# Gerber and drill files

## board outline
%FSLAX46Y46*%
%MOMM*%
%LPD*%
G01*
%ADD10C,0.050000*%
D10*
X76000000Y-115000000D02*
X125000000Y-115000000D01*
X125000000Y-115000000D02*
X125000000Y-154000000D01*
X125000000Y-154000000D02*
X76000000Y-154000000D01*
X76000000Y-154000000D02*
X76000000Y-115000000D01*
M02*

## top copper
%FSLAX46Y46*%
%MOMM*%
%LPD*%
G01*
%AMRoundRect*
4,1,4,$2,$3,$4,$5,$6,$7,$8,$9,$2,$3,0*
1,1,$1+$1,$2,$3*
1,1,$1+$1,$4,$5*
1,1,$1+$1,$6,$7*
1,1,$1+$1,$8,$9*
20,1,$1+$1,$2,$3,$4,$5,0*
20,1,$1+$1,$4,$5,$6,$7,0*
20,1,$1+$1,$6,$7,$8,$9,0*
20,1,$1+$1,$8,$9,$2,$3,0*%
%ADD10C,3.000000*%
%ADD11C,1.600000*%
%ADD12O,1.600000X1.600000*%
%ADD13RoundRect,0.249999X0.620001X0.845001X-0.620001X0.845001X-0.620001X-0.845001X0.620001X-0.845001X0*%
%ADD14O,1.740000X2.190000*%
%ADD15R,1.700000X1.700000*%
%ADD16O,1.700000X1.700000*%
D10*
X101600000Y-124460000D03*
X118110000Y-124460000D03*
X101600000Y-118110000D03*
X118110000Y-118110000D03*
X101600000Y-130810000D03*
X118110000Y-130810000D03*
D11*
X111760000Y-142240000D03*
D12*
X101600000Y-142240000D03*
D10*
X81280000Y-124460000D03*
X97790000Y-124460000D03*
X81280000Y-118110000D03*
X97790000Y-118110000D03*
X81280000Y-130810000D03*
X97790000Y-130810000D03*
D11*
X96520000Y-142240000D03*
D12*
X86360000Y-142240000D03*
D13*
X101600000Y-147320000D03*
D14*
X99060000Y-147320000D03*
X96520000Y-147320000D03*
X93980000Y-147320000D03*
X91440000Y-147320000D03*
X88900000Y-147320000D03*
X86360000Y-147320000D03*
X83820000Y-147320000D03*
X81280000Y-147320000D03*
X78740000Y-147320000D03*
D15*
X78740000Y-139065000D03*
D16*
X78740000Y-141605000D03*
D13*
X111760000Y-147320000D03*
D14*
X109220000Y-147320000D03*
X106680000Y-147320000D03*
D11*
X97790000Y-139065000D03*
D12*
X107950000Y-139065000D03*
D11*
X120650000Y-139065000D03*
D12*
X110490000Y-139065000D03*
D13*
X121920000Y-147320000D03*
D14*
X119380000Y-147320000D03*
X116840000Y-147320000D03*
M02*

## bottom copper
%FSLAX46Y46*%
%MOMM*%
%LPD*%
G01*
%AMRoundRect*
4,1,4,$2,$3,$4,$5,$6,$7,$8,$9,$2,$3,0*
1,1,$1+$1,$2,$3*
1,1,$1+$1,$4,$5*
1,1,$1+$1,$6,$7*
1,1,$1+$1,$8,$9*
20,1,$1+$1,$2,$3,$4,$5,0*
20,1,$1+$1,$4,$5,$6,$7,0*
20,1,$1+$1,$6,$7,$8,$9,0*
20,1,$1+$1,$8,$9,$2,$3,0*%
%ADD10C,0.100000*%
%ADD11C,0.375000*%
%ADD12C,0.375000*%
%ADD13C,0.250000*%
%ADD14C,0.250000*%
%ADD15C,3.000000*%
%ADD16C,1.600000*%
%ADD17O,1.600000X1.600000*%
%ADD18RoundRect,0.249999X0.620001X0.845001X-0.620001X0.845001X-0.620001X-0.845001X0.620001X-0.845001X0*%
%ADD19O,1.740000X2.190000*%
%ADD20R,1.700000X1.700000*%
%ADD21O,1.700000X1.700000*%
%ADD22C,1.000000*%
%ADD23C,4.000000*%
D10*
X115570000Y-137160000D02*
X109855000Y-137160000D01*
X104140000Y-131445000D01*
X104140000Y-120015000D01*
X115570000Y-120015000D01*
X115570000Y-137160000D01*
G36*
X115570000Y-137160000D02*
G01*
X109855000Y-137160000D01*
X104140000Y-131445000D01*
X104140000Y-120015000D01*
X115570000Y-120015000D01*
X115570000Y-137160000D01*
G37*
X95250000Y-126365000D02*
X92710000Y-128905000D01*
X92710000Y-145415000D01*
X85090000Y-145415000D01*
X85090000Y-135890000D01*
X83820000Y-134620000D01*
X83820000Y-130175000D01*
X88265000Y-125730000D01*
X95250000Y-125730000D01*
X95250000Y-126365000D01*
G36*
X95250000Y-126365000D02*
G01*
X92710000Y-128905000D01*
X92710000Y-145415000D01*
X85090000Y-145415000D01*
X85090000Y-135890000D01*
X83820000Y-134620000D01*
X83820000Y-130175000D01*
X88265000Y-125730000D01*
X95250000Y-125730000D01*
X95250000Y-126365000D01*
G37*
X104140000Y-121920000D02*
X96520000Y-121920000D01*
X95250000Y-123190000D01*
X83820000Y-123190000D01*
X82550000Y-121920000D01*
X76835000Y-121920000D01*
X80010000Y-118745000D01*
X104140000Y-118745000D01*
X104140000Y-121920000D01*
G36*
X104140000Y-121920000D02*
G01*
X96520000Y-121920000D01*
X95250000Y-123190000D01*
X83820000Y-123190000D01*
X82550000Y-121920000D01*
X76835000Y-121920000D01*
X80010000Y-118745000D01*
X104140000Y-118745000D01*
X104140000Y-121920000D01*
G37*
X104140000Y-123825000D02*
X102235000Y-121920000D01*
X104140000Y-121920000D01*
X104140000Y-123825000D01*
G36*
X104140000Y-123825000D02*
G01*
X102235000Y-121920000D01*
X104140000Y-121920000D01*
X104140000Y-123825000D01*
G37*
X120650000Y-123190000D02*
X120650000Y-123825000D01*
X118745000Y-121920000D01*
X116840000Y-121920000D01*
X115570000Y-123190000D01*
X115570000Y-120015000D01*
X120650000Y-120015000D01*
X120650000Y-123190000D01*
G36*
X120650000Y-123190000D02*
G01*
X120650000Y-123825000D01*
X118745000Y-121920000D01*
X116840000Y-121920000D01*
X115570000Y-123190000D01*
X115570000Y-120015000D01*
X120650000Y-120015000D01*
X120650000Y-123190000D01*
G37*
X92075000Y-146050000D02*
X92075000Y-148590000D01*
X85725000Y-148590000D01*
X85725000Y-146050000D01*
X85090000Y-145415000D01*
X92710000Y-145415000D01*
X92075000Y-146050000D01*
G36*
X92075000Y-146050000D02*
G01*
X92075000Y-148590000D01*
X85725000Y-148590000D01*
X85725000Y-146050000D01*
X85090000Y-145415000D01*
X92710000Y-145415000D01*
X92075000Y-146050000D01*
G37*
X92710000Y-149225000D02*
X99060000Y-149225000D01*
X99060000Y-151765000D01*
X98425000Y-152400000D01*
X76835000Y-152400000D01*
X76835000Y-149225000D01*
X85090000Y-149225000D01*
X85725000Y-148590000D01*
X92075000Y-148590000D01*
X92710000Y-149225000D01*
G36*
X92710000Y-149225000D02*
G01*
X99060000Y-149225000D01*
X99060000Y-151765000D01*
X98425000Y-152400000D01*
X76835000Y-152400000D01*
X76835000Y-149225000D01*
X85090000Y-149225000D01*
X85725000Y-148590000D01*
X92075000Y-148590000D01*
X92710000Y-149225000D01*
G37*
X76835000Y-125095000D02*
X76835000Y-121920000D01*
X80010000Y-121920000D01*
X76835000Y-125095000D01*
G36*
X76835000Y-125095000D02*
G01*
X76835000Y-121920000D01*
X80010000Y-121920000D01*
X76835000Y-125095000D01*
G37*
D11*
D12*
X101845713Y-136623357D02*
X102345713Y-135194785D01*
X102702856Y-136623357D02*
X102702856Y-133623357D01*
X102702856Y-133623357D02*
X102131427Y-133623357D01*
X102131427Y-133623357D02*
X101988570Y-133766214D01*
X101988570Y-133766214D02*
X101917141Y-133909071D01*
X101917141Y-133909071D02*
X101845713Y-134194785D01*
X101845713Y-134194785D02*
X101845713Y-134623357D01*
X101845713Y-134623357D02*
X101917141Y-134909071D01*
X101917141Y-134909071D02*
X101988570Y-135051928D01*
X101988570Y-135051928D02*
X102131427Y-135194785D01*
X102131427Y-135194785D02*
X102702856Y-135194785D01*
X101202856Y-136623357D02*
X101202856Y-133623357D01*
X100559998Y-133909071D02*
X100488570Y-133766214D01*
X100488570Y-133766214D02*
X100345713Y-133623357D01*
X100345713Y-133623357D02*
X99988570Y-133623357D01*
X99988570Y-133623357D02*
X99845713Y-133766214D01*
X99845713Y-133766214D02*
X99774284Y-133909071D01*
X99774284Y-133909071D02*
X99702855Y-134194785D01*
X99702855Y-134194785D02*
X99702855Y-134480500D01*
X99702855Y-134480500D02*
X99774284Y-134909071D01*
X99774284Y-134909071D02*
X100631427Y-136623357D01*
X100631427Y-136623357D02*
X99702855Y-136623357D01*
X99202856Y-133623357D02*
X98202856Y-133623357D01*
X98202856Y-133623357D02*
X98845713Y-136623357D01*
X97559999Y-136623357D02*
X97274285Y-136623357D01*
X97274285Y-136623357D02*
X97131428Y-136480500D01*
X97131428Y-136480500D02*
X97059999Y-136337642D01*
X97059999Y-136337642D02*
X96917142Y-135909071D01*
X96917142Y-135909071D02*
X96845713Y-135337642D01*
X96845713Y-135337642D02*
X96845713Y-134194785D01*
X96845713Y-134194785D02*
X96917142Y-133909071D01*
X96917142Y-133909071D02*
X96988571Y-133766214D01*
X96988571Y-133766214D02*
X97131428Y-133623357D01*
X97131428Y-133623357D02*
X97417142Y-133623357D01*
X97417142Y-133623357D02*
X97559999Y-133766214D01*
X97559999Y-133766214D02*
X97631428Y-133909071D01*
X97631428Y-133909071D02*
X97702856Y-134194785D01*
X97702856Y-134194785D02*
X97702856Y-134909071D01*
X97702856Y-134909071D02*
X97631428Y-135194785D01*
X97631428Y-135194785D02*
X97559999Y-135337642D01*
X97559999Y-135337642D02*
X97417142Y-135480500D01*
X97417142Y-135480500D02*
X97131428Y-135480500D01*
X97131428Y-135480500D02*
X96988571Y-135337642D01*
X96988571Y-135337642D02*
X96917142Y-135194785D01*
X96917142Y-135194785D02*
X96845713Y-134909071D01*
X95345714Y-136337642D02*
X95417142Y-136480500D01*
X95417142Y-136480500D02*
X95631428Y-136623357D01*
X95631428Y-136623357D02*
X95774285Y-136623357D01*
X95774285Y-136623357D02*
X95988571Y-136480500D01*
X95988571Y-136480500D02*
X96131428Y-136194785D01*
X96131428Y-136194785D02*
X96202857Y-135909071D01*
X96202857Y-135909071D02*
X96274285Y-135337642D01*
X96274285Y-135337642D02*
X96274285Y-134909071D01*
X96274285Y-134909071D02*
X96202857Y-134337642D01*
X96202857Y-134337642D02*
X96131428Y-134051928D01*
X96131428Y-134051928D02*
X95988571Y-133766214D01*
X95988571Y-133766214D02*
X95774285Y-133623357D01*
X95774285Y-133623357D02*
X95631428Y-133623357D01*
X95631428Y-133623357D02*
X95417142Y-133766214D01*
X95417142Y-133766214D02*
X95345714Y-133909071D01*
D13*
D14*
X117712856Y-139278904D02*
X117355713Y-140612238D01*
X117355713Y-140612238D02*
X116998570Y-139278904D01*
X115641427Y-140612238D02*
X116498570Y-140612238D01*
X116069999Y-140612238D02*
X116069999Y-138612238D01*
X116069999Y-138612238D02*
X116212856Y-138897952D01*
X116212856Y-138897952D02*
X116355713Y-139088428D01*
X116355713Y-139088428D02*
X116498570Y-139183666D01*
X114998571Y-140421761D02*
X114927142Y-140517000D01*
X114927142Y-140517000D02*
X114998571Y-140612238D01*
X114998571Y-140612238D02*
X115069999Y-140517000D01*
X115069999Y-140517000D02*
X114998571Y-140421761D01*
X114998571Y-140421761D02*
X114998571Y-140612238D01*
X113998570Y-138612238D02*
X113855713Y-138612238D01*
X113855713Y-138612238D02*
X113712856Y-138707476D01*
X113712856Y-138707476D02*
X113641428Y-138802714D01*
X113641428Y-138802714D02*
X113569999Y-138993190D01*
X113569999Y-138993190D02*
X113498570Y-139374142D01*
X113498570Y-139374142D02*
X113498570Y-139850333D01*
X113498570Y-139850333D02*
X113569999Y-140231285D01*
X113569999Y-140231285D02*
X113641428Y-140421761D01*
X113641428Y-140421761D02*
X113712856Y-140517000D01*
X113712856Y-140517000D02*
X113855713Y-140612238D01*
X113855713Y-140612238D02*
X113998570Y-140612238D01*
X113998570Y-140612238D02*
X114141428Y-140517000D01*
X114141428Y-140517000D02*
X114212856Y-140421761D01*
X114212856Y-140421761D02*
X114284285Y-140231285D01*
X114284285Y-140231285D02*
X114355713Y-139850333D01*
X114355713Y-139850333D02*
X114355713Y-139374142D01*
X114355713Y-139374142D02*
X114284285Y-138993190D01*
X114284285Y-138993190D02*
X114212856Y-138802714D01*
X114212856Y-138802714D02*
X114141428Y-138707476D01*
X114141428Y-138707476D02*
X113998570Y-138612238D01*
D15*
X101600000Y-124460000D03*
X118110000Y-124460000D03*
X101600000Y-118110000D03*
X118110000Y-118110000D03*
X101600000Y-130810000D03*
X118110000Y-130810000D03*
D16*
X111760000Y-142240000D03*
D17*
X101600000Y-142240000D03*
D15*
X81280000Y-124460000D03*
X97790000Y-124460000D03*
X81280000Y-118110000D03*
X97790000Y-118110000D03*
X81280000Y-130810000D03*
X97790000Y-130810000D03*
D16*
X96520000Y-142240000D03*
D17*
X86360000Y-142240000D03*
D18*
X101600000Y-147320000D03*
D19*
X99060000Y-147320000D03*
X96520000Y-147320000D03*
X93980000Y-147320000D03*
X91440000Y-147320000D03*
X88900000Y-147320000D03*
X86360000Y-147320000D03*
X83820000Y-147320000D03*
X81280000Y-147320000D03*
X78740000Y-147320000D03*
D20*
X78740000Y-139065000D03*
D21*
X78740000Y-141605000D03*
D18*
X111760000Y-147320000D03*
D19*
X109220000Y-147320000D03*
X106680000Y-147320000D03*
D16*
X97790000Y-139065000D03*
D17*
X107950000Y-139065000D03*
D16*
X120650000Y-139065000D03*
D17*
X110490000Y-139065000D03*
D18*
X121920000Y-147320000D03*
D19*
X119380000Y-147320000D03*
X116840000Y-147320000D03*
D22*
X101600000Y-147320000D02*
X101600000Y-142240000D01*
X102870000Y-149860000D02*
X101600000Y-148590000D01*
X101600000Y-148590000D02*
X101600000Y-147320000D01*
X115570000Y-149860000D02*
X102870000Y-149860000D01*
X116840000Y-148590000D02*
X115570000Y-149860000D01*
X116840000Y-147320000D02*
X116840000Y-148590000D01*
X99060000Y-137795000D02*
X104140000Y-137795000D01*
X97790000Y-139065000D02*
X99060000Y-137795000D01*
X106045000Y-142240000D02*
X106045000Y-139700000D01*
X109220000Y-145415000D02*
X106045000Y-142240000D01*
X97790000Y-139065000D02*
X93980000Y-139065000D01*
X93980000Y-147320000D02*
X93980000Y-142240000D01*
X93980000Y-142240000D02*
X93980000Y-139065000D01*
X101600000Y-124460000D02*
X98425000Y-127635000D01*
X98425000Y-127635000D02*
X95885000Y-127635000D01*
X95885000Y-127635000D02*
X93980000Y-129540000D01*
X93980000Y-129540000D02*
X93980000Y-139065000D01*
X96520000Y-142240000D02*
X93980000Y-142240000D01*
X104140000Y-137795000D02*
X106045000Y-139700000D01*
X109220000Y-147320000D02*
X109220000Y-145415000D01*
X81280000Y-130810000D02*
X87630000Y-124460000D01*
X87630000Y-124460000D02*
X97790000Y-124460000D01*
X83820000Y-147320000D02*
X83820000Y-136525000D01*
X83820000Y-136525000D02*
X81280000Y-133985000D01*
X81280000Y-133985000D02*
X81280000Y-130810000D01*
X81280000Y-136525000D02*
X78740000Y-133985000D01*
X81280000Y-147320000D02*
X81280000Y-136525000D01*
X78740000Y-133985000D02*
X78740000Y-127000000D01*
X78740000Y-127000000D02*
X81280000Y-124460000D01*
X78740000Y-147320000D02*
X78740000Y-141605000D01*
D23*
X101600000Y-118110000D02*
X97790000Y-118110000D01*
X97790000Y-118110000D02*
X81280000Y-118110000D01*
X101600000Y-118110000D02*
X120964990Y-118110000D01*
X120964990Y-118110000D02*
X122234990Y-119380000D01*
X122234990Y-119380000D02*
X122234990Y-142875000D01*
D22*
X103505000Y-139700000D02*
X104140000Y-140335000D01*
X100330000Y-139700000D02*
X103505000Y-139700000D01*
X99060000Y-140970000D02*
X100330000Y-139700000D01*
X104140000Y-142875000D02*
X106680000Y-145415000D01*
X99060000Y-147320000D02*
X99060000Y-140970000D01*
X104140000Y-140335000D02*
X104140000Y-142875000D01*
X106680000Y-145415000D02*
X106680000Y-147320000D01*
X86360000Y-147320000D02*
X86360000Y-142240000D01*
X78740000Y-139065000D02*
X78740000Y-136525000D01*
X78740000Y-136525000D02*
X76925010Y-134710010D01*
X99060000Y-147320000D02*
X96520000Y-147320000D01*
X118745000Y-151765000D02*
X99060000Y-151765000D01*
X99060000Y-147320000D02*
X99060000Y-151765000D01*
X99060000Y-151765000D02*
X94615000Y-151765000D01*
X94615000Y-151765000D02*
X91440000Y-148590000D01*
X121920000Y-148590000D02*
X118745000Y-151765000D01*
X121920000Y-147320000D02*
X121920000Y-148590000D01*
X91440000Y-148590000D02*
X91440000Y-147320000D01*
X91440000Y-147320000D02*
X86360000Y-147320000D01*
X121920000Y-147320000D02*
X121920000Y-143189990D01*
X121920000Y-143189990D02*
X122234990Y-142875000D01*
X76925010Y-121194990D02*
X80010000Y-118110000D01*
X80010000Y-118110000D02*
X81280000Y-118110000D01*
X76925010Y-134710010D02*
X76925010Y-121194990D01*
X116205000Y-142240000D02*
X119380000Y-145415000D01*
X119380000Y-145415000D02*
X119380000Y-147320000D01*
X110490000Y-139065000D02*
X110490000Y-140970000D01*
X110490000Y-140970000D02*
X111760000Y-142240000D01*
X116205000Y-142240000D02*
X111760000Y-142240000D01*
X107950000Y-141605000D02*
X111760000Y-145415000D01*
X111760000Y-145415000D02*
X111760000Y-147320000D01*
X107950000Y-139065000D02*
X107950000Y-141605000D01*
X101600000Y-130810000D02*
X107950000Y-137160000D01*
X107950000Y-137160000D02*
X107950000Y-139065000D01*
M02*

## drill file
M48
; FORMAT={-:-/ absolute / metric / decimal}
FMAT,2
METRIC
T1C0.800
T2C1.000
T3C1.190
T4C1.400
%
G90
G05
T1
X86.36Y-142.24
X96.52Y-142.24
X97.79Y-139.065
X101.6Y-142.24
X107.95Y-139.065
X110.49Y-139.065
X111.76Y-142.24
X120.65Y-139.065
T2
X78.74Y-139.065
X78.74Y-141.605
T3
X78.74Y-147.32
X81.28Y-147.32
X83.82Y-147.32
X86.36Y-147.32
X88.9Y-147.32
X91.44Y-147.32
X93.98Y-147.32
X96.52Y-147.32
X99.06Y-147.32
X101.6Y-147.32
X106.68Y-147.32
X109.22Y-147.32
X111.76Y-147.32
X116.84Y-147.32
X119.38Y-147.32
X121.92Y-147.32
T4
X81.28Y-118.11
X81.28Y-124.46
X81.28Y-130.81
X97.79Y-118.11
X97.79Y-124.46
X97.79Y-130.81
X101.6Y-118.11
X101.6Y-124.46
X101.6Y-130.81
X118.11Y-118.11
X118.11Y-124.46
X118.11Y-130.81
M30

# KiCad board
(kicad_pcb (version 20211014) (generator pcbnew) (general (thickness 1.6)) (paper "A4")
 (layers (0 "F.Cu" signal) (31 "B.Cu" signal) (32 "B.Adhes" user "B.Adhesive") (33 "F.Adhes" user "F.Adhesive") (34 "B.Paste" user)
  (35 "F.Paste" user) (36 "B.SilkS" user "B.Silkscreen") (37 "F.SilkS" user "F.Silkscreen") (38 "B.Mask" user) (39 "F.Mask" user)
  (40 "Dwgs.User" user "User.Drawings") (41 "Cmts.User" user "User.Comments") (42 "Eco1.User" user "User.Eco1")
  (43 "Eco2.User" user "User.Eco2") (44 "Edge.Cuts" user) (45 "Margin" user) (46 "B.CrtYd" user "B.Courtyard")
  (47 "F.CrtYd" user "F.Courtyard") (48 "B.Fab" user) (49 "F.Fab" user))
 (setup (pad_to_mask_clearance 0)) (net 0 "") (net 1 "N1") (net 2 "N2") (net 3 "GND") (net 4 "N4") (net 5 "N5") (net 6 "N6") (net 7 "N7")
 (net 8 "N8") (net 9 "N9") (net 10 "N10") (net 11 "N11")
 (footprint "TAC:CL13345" (layer "F.Cu") (at 109.855 118.11 90)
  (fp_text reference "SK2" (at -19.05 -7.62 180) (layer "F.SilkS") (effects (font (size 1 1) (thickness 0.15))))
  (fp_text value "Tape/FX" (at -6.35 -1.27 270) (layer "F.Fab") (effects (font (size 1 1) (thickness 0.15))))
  (pad "R" thru_hole circle locked (at -6.35 -8.255 180) (size 3 3) (drill 1.4) (layers *.Cu *.Mask) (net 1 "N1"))
  (pad "RN" thru_hole circle locked (at -6.35 8.255 180) (size 3 3) (drill 1.4) (layers *.Cu *.Mask) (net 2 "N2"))
  (pad "S" thru_hole circle locked (at 0 -8.255 180) (size 3 3) (drill 1.4) (layers *.Cu *.Mask) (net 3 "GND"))
  (pad "SN" thru_hole circle locked (at 0 8.255 180) (size 3 3) (drill 1.4) (layers *.Cu *.Mask) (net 3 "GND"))
  (pad "T" thru_hole circle locked (at -12.7 -8.255 180) (size 3 3) (drill 1.4) (layers *.Cu *.Mask) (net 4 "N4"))
  (pad "TN" thru_hole circle locked (at -12.7 8.255 180) (size 3 3) (drill 1.4) (layers *.Cu *.Mask) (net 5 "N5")))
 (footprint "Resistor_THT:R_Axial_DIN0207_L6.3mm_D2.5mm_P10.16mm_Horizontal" (layer "F.Cu") (at 111.76 142.24 180)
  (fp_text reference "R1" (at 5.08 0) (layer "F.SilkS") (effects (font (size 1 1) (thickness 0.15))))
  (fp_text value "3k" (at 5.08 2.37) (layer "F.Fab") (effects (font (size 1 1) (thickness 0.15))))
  (pad "1" thru_hole circle locked (at 0 0 180) (size 1.6 1.6) (drill 0.8) (layers *.Cu *.Mask) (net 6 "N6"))
  (pad "2" thru_hole oval locked (at 10.16 0 180) (size 1.6 1.6) (drill 0.8) (layers *.Cu *.Mask) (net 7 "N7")))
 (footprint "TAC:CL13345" (layer "F.Cu") (at 89.535 118.11 90)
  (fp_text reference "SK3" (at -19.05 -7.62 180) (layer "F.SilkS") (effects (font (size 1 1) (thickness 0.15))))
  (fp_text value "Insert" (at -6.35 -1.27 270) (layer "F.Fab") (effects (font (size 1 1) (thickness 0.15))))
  (pad "R" thru_hole circle locked (at -6.35 -8.255 180) (size 3 3) (drill 1.4) (layers *.Cu *.Mask) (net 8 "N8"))
  (pad "RN" thru_hole circle locked (at -6.35 8.255 180) (size 3 3) (drill 1.4) (layers *.Cu *.Mask) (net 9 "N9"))
  (pad "S" thru_hole circle locked (at 0 -8.255 180) (size 3 3) (drill 1.4) (layers *.Cu *.Mask) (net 3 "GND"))
  (pad "SN" thru_hole circle locked (at 0 8.255 180) (size 3 3) (drill 1.4) (layers *.Cu *.Mask) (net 3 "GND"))
  (pad "T" thru_hole circle locked (at -12.7 -8.255 180) (size 3 3) (drill 1.4) (layers *.Cu *.Mask) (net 9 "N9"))
  (pad "TN" thru_hole circle locked (at -12.7 8.255 180) (size 3 3) (drill 1.4) (layers *.Cu *.Mask) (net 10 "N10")))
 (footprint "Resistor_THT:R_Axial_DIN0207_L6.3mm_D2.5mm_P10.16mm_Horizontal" (layer "F.Cu") (at 96.52 142.24 180)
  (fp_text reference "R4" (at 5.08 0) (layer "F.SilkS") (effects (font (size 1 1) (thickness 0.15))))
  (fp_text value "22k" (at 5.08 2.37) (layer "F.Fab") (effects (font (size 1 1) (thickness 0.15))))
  (pad "1" thru_hole circle locked (at 0 0 180) (size 1.6 1.6) (drill 0.8) (layers *.Cu *.Mask) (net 1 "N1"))
  (pad "2" thru_hole oval locked (at 10.16 0 180) (size 1.6 1.6) (drill 0.8) (layers *.Cu *.Mask) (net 3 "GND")))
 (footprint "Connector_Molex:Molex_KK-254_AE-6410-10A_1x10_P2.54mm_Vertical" (layer "F.Cu") (at 101.6 147.32 180)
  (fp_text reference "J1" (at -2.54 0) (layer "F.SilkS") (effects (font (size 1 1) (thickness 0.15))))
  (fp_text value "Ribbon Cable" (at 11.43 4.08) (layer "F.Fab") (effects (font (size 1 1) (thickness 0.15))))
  (pad "1" thru_hole roundrect locked (at 0 0 180) (size 1.74 2.19) (drill 1.19) (layers *.Cu *.Mask) (roundrect_rratio 0.1436775862)
   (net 7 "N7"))
  (pad "2" thru_hole oval locked (at 2.54 0 180) (size 1.74 2.19) (drill 1.19) (layers *.Cu *.Mask) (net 3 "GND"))
  (pad "3" thru_hole oval locked (at 5.08 0 180) (size 1.74 2.19) (drill 1.19) (layers *.Cu *.Mask) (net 3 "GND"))
  (pad "4" thru_hole oval locked (at 7.62 0 180) (size 1.74 2.19) (drill 1.19) (layers *.Cu *.Mask) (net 1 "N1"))
  (pad "5" thru_hole oval locked (at 10.16 0 180) (size 1.74 2.19) (drill 1.19) (layers *.Cu *.Mask) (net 3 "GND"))
  (pad "6" thru_hole oval locked (at 12.7 0 180) (size 1.74 2.19) (drill 1.19) (layers *.Cu *.Mask) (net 3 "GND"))
  (pad "7" thru_hole oval locked (at 15.24 0 180) (size 1.74 2.19) (drill 1.19) (layers *.Cu *.Mask) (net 3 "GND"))
  (pad "8" thru_hole oval locked (at 17.78 0 180) (size 1.74 2.19) (drill 1.19) (layers *.Cu *.Mask) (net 9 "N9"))
  (pad "9" thru_hole oval locked (at 20.32 0 180) (size 1.74 2.19) (drill 1.19) (layers *.Cu *.Mask) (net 8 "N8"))
  (pad "10" thru_hole oval locked (at 22.86 0 180) (size 1.74 2.19) (drill 1.19) (layers *.Cu *.Mask) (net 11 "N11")))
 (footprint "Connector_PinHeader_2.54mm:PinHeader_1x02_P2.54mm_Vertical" (layer "F.Cu") (at 78.74 139.065)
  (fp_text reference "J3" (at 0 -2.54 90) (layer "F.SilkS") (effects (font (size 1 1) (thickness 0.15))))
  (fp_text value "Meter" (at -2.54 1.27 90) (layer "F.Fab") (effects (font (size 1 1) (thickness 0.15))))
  (pad "1" thru_hole rect locked (at 0 0) (size 1.7 1.7) (drill 1) (layers *.Cu *.Mask) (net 3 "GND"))
  (pad "2" thru_hole oval locked (at 0 2.54) (size 1.7 1.7) (drill 1) (layers *.Cu *.Mask) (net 11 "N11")))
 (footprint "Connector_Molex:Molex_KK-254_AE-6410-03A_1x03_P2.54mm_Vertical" (layer "F.Cu") (at 111.76 147.32 180)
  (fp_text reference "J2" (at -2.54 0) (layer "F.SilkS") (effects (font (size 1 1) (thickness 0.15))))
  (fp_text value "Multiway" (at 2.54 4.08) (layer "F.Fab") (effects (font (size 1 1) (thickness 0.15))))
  (pad "1" thru_hole roundrect locked (at 0 0 180) (size 1.74 2.19) (drill 1.19) (layers *.Cu *.Mask) (roundrect_rratio 0.1436775862)
   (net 4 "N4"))
  (pad "2" thru_hole oval locked (at 2.54 0 180) (size 1.74 2.19) (drill 1.19) (layers *.Cu *.Mask) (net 1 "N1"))
  (pad "3" thru_hole oval locked (at 5.08 0 180) (size 1.74 2.19) (drill 1.19) (layers *.Cu *.Mask) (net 3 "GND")))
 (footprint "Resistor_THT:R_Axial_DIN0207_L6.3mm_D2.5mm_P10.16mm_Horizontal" (layer "F.Cu") (at 97.79 139.065)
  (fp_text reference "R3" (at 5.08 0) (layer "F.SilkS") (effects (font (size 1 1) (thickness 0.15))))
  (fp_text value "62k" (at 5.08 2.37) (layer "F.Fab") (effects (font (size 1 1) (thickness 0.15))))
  (pad "1" thru_hole circle locked (at 0 0) (size 1.6 1.6) (drill 0.8) (layers *.Cu *.Mask) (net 1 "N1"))
  (pad "2" thru_hole oval locked (at 10.16 0) (size 1.6 1.6) (drill 0.8) (layers *.Cu *.Mask) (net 4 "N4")))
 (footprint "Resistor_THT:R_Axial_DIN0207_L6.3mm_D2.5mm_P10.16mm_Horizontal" (layer "F.Cu") (at 120.65 139.065 180)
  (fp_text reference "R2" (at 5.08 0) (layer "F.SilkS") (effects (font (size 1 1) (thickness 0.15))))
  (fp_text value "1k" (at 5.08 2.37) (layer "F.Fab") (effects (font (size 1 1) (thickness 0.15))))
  (pad "1" thru_hole circle locked (at 0 0 180) (size 1.6 1.6) (drill 0.8) (layers *.Cu *.Mask) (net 3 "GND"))
  (pad "2" thru_hole oval locked (at 10.16 0 180) (size 1.6 1.6) (drill 0.8) (layers *.Cu *.Mask) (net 6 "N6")))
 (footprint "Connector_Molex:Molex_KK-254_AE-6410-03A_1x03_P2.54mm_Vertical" (layer "F.Cu") (at 121.92 147.32 180)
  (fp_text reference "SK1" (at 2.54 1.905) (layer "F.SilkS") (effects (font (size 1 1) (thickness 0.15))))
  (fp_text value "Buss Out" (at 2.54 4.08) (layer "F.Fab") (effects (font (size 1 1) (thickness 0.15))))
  (pad "1" thru_hole roundrect locked (at 0 0 180) (size 1.74 2.19) (drill 1.19) (layers *.Cu *.Mask) (roundrect_rratio 0.1436775862)
   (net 3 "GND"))
  (pad "2" thru_hole oval locked (at 2.54 0 180) (size 1.74 2.19) (drill 1.19) (layers *.Cu *.Mask) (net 6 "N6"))
  (pad "3" thru_hole oval locked (at 5.08 0 180) (size 1.74 2.19) (drill 1.19) (layers *.Cu *.Mask) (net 7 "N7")))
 (gr_poly
  (pts (xy 115.57 137.16) (xy 109.855 137.16) (xy 104.14 131.445) (xy 104.14 120.015) (xy 115.57 120.015)) (layer "B.Cu") (width 0.1)
  (fill solid))
 (gr_poly
  (pts (xy 95.25 126.365) (xy 92.71 128.905) (xy 92.71 145.415) (xy 85.09 145.415) (xy 85.09 135.89) (xy 83.82 134.62) (xy 83.82 130.175)
   (xy 88.265 125.73) (xy 95.25 125.73))
  (layer "B.Cu") (width 0.1) (fill solid))
 (gr_poly
  (pts (xy 104.14 121.92) (xy 96.52 121.92) (xy 95.25 123.19) (xy 83.82 123.19) (xy 82.55 121.92) (xy 76.835 121.92) (xy 80.01 118.745)
   (xy 104.14 118.745))
  (layer "B.Cu") (width 0.1) (fill solid))
 (gr_poly (pts (xy 104.14 123.825) (xy 102.235 121.92) (xy 104.14 121.92)) (layer "B.Cu") (width 0.1) (fill solid))
 (gr_poly
  (pts (xy 120.65 123.19) (xy 120.65 123.825) (xy 118.745 121.92) (xy 116.84 121.92) (xy 115.57 123.19) (xy 115.57 120.015)
   (xy 120.65 120.015))
  (layer "B.Cu") (width 0.1) (fill solid))
 (gr_poly
  (pts (xy 92.075 146.05) (xy 92.075 148.59) (xy 85.725 148.59) (xy 85.725 146.05) (xy 85.09 145.415) (xy 92.71 145.415)) (layer "B.Cu")
  (width 0.1) (fill solid))
 (gr_poly
  (pts (xy 92.71 149.225) (xy 99.06 149.225) (xy 99.06 151.765) (xy 98.425 152.4) (xy 76.835 152.4) (xy 76.835 149.225) (xy 85.09 149.225)
   (xy 85.725 148.59) (xy 92.075 148.59))
  (layer "B.Cu") (width 0.1) (fill solid))
 (gr_poly (pts (xy 76.835 125.095) (xy 76.835 121.92) (xy 80.01 121.92)) (layer "B.Cu") (width 0.1) (fill solid))
 (gr_line (start 76 115) (end 125 115) (layer "Edge.Cuts") (width 0.05))
 (gr_line (start 125 115) (end 125 154) (layer "Edge.Cuts") (width 0.05))
 (gr_line (start 125 154) (end 76 154) (layer "Edge.Cuts") (width 0.05))
 (gr_line (start 76 154) (end 76 115) (layer "Edge.Cuts") (width 0.05))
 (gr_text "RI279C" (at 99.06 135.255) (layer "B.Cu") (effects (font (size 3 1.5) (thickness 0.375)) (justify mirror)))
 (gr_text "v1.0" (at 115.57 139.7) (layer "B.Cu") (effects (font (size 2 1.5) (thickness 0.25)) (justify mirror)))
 (segment (start 101.6 147.32) (end 101.6 142.24) (width 1) (layer "B.Cu") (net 7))
 (segment (start 102.87 149.86) (end 101.6 148.59) (width 1) (layer "B.Cu") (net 7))
 (segment (start 101.6 148.59) (end 101.6 147.32) (width 1) (layer "B.Cu") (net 7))
 (segment (start 115.57 149.86) (end 102.87 149.86) (width 1) (layer "B.Cu") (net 7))
 (segment (start 116.84 148.59) (end 115.57 149.86) (width 1) (layer "B.Cu") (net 7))
 (segment (start 116.84 147.32) (end 116.84 148.59) (width 1) (layer "B.Cu") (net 7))
 (segment (start 99.06 137.795) (end 104.14 137.795) (width 1) (layer "B.Cu") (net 1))
 (segment (start 97.79 139.065) (end 99.06 137.795) (width 1) (layer "B.Cu") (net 1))
 (segment (start 106.045 142.24) (end 106.045 139.7) (width 1) (layer "B.Cu") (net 1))
 (segment (start 109.22 145.415) (end 106.045 142.24) (width 1) (layer "B.Cu") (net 1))
 (segment (start 97.79 139.065) (end 93.98 139.065) (width 1) (layer "B.Cu") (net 1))
 (segment (start 93.98 147.32) (end 93.98 142.24) (width 1) (layer "B.Cu") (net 1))
 (segment (start 93.98 142.24) (end 93.98 139.065) (width 1) (layer "B.Cu") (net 1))
 (segment (start 101.6 124.46) (end 98.425 127.635) (width 1) (layer "B.Cu") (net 1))
 (segment (start 98.425 127.635) (end 95.885 127.635) (width 1) (layer "B.Cu") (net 1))
 (segment (start 95.885 127.635) (end 93.98 129.54) (width 1) (layer "B.Cu") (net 1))
 (segment (start 93.98 129.54) (end 93.98 139.065) (width 1) (layer "B.Cu") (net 1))
 (segment (start 96.52 142.24) (end 93.98 142.24) (width 1) (layer "B.Cu") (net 1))
 (segment (start 104.14 137.795) (end 106.045 139.7) (width 1) (layer "B.Cu") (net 1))
 (segment (start 109.22 147.32) (end 109.22 145.415) (width 1) (layer "B.Cu") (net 1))
 (segment (start 81.28 130.81) (end 87.63 124.46) (width 1) (layer "B.Cu") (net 9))
 (segment (start 87.63 124.46) (end 97.79 124.46) (width 1) (layer "B.Cu") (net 9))
 (segment (start 83.82 147.32) (end 83.82 136.525) (width 1) (layer "B.Cu") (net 9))
 (segment (start 83.82 136.525) (end 81.28 133.985) (width 1) (layer "B.Cu") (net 9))
 (segment (start 81.28 133.985) (end 81.28 130.81) (width 1) (layer "B.Cu") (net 9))
 (segment (start 81.28 136.525) (end 78.74 133.985) (width 1) (layer "B.Cu") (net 8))
 (segment (start 81.28 147.32) (end 81.28 136.525) (width 1) (layer "B.Cu") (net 8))
 (segment (start 78.74 133.985) (end 78.74 127) (width 1) (layer "B.Cu") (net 8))
 (segment (start 78.74 127) (end 81.28 124.46) (width 1) (layer "B.Cu") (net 8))
 (segment (start 78.74 147.32) (end 78.74 141.605) (width 1) (layer "B.Cu") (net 11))
 (segment (start 101.6 118.11) (end 97.79 118.11) (width 4) (layer "B.Cu") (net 3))
 (segment (start 97.79 118.11) (end 81.28 118.11) (width 4) (layer "B.Cu") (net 3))
 (segment (start 101.6 118.11) (end 120.96499 118.11) (width 4) (layer "B.Cu") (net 3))
 (segment (start 120.96499 118.11) (end 122.23499 119.38) (width 4) (layer "B.Cu") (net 3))
 (segment (start 122.23499 119.38) (end 122.23499 142.875) (width 4) (layer "B.Cu") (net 3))
 (segment (start 103.505 139.7) (end 104.14 140.335) (width 1) (layer "B.Cu") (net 3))
 (segment (start 100.33 139.7) (end 103.505 139.7) (width 1) (layer "B.Cu") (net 3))
 (segment (start 99.06 140.97) (end 100.33 139.7) (width 1) (layer "B.Cu") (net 3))
 (segment (start 104.14 142.875) (end 106.68 145.415) (width 1) (layer "B.Cu") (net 3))
 (segment (start 99.06 147.32) (end 99.06 140.97) (width 1) (layer "B.Cu") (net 3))
 (segment (start 104.14 140.335) (end 104.14 142.875) (width 1) (layer "B.Cu") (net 3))
 (segment (start 106.68 145.415) (end 106.68 147.32) (width 1) (layer "B.Cu") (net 3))
 (segment (start 86.36 147.32) (end 86.36 142.24) (width 1) (layer "B.Cu") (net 3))
 (segment (start 78.74 139.065) (end 78.74 136.525) (width 1) (layer "B.Cu") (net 3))
 (segment (start 78.74 136.525) (end 76.92501 134.71001) (width 1) (layer "B.Cu") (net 3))
 (segment (start 99.06 147.32) (end 96.52 147.32) (width 1) (layer "B.Cu") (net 3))
 (segment (start 118.745 151.765) (end 99.06 151.765) (width 1) (layer "B.Cu") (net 3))
 (segment (start 99.06 147.32) (end 99.06 151.765) (width 1) (layer "B.Cu") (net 3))
 (segment (start 99.06 151.765) (end 94.615 151.765) (width 1) (layer "B.Cu") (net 3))
 (segment (start 94.615 151.765) (end 91.44 148.59) (width 1) (layer "B.Cu") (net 3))
 (segment (start 121.92 148.59) (end 118.745 151.765) (width 1) (layer "B.Cu") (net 3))
 (segment (start 121.92 147.32) (end 121.92 148.59) (width 1) (layer "B.Cu") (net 3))
 (segment (start 91.44 148.59) (end 91.44 147.32) (width 1) (layer "B.Cu") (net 3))
 (segment (start 91.44 147.32) (end 86.36 147.32) (width 1) (layer "B.Cu") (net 3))
 (segment (start 121.92 147.32) (end 121.92 143.18999) (width 1) (layer "B.Cu") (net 3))
 (segment (start 121.92 143.18999) (end 122.23499 142.875) (width 1) (layer "B.Cu") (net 3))
 (segment (start 76.92501 121.19499) (end 80.01 118.11) (width 1) (layer "B.Cu") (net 3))
 (segment (start 80.01 118.11) (end 81.28 118.11) (width 1) (layer "B.Cu") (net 3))
 (segment (start 76.92501 134.71001) (end 76.92501 121.19499) (width 1) (layer "B.Cu") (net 3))
 (segment (start 116.205 142.24) (end 119.38 145.415) (width 1) (layer "B.Cu") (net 6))
 (segment (start 119.38 145.415) (end 119.38 147.32) (width 1) (layer "B.Cu") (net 6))
 (segment (start 110.49 139.065) (end 110.49 140.97) (width 1) (layer "B.Cu") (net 6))
 (segment (start 110.49 140.97) (end 111.76 142.24) (width 1) (layer "B.Cu") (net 6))
 (segment (start 116.205 142.24) (end 111.76 142.24) (width 1) (layer "B.Cu") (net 6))
 (segment (start 107.95 141.605) (end 111.76 145.415) (width 1) (layer "B.Cu") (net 4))
 (segment (start 111.76 145.415) (end 111.76 147.32) (width 1) (layer "B.Cu") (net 4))
 (segment (start 107.95 139.065) (end 107.95 141.605) (width 1) (layer "B.Cu") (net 4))
 (segment (start 101.6 130.81) (end 107.95 137.16) (width 1) (layer "B.Cu") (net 4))
 (segment (start 107.95 137.16) (end 107.95 139.065) (width 1) (layer "B.Cu") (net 4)))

